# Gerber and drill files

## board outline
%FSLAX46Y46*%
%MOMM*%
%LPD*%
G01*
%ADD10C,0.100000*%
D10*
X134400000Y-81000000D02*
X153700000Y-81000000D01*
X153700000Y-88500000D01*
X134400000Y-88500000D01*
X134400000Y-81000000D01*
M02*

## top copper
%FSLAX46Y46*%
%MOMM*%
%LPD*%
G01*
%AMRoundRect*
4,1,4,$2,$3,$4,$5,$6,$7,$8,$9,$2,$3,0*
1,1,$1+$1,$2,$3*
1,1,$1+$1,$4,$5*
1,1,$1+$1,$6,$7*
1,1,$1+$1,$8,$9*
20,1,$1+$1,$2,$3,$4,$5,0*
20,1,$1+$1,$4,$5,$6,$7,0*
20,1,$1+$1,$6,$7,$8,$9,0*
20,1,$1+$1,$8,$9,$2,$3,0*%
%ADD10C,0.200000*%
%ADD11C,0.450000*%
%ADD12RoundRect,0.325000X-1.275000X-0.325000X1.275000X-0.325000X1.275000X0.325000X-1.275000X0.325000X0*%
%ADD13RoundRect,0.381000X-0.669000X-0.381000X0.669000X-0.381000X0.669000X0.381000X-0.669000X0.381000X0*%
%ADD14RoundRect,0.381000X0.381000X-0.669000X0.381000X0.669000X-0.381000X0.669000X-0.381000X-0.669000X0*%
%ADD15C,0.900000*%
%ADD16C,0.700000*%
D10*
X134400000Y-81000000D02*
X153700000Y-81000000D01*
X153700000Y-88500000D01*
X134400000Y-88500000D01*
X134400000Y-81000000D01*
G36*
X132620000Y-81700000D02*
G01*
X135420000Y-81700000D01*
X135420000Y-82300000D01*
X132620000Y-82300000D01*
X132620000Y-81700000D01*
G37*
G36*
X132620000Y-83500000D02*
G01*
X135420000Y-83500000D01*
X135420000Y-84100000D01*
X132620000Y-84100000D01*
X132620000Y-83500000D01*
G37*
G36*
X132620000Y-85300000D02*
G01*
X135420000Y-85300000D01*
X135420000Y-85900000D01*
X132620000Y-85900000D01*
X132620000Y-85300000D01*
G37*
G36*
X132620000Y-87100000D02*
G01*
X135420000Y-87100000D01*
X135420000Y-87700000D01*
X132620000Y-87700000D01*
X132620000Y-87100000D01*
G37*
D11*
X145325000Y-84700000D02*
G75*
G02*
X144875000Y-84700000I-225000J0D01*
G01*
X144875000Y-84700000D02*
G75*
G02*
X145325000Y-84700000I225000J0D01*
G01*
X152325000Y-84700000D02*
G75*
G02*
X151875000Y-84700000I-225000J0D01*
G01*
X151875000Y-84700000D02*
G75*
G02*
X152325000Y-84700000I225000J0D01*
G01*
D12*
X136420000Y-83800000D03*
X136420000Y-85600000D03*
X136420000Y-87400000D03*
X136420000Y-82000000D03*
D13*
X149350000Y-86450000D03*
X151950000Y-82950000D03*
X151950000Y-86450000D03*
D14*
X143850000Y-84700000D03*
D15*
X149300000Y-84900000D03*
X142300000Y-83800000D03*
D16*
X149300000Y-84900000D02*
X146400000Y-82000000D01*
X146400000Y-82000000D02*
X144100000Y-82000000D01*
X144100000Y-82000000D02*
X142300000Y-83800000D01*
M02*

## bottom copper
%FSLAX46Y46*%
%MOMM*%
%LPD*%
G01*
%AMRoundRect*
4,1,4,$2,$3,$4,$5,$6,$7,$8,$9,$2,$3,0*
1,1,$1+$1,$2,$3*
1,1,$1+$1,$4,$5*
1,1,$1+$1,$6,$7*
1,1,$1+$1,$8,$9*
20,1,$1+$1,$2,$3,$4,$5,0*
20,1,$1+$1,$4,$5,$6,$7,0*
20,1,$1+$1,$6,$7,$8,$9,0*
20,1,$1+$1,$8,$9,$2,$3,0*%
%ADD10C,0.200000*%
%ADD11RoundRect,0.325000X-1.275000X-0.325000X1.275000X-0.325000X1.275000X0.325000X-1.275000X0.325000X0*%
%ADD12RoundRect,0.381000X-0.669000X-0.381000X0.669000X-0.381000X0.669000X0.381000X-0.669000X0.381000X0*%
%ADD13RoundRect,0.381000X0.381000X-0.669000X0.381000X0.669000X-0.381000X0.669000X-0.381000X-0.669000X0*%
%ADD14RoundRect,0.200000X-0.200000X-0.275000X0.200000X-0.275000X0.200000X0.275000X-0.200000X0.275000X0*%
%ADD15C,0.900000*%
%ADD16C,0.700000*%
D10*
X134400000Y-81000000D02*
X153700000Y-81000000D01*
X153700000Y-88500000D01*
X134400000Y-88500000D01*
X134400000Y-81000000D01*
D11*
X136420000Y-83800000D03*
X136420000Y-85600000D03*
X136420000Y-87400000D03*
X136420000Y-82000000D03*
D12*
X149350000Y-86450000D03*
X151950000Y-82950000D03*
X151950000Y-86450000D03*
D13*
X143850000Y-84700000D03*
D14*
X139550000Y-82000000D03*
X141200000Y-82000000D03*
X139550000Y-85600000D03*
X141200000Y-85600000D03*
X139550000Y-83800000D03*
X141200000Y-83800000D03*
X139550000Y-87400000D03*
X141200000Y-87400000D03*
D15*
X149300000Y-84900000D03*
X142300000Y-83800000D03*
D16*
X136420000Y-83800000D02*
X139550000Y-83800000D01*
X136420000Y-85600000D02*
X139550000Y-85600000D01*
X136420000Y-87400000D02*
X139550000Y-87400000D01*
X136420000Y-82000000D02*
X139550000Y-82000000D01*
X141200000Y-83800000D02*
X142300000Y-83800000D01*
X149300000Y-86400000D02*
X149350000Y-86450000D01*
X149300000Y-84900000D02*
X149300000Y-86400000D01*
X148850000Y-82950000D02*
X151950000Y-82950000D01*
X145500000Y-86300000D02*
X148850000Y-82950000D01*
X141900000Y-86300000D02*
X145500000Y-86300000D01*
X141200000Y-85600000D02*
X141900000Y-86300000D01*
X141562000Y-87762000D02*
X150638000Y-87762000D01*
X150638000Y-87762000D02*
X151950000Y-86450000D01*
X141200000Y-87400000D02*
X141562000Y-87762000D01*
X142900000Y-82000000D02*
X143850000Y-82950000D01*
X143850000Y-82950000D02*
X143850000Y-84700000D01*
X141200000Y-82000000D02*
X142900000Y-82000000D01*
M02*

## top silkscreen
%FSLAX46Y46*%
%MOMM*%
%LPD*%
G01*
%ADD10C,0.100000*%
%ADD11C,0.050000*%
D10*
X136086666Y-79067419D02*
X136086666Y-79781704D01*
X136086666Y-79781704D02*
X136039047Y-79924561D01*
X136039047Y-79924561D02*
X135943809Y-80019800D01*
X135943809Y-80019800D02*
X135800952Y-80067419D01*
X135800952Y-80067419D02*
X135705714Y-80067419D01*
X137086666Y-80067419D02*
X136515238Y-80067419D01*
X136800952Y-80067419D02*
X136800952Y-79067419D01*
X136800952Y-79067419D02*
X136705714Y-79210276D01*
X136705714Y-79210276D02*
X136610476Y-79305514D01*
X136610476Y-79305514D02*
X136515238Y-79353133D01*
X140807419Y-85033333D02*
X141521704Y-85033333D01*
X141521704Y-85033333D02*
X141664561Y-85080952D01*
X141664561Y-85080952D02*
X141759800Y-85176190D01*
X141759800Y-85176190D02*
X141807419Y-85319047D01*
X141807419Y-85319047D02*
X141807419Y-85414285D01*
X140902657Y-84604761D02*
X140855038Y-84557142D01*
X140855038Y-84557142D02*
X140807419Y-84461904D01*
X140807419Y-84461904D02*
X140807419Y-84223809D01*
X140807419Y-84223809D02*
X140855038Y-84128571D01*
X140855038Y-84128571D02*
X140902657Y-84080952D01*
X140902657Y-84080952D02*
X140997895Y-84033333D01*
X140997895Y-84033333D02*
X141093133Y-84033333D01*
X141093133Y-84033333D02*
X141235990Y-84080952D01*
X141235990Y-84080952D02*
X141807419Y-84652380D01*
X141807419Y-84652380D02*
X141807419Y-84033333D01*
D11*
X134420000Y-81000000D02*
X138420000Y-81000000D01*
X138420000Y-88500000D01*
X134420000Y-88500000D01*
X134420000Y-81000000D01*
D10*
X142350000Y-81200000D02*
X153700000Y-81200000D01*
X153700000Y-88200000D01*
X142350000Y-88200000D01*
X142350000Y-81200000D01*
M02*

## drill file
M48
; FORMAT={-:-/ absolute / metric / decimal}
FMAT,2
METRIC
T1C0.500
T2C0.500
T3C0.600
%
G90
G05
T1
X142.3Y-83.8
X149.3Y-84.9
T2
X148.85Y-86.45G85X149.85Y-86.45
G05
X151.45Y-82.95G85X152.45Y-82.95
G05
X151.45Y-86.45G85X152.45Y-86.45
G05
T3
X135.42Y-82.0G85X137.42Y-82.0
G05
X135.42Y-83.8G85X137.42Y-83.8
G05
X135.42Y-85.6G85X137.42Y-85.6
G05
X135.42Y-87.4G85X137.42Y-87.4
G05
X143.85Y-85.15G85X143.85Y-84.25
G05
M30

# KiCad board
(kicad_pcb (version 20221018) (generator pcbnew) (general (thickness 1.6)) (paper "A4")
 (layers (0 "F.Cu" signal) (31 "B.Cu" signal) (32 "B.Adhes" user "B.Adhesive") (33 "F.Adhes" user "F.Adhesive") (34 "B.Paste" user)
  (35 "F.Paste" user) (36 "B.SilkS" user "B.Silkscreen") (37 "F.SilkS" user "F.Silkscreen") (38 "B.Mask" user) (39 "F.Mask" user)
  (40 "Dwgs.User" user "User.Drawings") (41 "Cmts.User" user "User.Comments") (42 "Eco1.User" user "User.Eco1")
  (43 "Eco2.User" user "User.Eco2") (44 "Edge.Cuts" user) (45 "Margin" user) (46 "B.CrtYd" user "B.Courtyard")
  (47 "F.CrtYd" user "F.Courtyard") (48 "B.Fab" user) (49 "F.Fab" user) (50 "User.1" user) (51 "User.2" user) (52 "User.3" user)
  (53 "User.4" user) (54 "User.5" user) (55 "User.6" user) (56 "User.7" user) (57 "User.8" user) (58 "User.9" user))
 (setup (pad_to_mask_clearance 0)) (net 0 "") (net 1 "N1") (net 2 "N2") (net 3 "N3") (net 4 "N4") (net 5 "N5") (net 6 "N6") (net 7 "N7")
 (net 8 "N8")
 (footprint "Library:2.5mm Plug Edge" (layer "F.Cu") (at 136.42 88.5)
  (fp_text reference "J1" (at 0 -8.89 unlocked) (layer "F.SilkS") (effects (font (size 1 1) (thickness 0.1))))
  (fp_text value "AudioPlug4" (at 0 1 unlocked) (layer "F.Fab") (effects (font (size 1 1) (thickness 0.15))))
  (fp_rect (start -3.8 -6.8) (end -1 -6.2) (stroke (width 0) (type solid)) (fill solid) (layer "F.Cu"))
  (fp_rect (start -3.8 -5) (end -1 -4.4) (stroke (width 0) (type solid)) (fill solid) (layer "F.Cu"))
  (fp_rect (start -3.8 -3.2) (end -1 -2.6) (stroke (width 0) (type solid)) (fill solid) (layer "F.Cu"))
  (fp_rect (start -3.8 -1.4) (end -1 -0.8) (stroke (width 0) (type solid)) (fill solid) (layer "F.Cu"))
  (fp_rect (start -2 -7.5) (end 2 0) (stroke (width 0.05) (type default)) (fill none) (layer "F.SilkS"))
  (pad "R1" thru_hole roundrect (at 0 -4.7) (size 3.2 1.3) (drill oval 2.6 0.6) (layers "*.Cu" "*.Mask") (roundrect_rratio 0.25)
   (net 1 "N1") (thermal_bridge_angle 45))
  (pad "R2" thru_hole roundrect (at 0 -2.9) (size 3.2 1.3) (drill oval 2.6 0.6) (layers "*.Cu" "*.Mask") (roundrect_rratio 0.25)
   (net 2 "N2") (thermal_bridge_angle 45))
  (pad "S" thru_hole roundrect (at 0 -1.1) (size 3.2 1.3) (drill oval 2.6 0.6) (layers "*.Cu" "*.Mask") (roundrect_rratio 0.25) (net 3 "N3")
   (thermal_bridge_angle 45))
  (pad "T" thru_hole roundrect (at 0 -6.5) (size 3.2 1.3) (drill oval 2.6 0.6) (layers "*.Cu" "*.Mask") (roundrect_rratio 0.25) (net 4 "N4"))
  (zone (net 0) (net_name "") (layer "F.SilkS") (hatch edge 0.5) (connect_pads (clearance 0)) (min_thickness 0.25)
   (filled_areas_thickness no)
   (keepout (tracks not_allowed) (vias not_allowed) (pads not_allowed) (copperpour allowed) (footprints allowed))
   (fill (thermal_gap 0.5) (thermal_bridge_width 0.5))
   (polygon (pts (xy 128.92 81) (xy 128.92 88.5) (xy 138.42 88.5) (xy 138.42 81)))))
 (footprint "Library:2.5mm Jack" (layer "F.Cu") (at 153.85 84.7 90)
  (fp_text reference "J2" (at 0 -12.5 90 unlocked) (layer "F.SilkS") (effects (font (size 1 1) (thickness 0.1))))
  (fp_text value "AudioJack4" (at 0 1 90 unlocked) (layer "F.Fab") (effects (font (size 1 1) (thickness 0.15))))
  (fp_circle (center 0 -8.75) (end 0.4 -8.75) (stroke (width 0.1) (type solid)) (fill solid) (layer "F.Cu"))
  (fp_circle (center 0 -1.75) (end 0.4 -1.75) (stroke (width 0.1) (type solid)) (fill solid) (layer "F.Cu"))
  (fp_rect (start -3.5 -11.5) (end 3.5 -0.15) (stroke (width 0.1) (type default)) (fill none) (layer "F.SilkS"))
  (pad "R1" thru_hole roundrect (at -1.75 -4.5) (size 2.1 1.524) (drill oval 1.5 0.5) (layers "*.Cu" "*.Mask") (roundrect_rratio 0.25)
   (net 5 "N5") (thermal_bridge_angle 45))
  (pad "R2" thru_hole roundrect (at 1.75 -1.9) (size 2.1 1.524) (drill oval 1.5 0.5) (layers "*.Cu" "*.Mask") (roundrect_rratio 0.25)
   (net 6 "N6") (thermal_bridge_angle 45))
  (pad "S" thru_hole roundrect (at -1.75 -1.9) (size 2.1 1.524) (drill oval 1.5 0.5) (layers "*.Cu" "*.Mask") (roundrect_rratio 0.25)
   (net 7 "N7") (thermal_bridge_angle 45))
  (pad "T" thru_hole roundrect (at 0 -10 90) (size 2.1 1.524) (drill oval 1.5 0.6) (layers "*.Cu" "*.Mask") (roundrect_rratio 0.25)
   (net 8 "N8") (thermal_bridge_angle 45))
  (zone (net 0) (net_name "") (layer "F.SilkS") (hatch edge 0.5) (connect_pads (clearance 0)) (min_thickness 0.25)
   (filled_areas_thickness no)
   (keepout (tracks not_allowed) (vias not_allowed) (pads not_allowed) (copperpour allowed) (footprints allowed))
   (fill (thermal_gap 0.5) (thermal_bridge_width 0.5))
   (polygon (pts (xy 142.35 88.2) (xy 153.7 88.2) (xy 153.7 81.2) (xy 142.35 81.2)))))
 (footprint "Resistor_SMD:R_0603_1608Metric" (layer "B.Cu") (at 140.375 82)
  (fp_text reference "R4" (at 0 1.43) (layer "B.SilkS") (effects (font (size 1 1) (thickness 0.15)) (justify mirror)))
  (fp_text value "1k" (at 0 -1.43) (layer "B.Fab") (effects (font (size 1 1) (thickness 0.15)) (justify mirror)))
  (pad "1" smd roundrect (at -0.825 0) (size 0.8 0.95) (layers "B.Cu" "B.Paste" "B.Mask") (roundrect_rratio 0.25) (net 4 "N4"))
  (pad "2" smd roundrect (at 0.825 0) (size 0.8 0.95) (layers "B.Cu" "B.Paste" "B.Mask") (roundrect_rratio 0.25) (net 8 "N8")))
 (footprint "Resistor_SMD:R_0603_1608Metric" (layer "B.Cu") (at 140.375 85.6)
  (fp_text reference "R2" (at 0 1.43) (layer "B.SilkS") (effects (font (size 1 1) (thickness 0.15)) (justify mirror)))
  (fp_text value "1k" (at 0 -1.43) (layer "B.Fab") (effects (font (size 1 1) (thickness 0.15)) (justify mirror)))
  (pad "1" smd roundrect (at -0.825 0) (size 0.8 0.95) (layers "B.Cu" "B.Paste" "B.Mask") (roundrect_rratio 0.25) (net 2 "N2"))
  (pad "2" smd roundrect (at 0.825 0) (size 0.8 0.95) (layers "B.Cu" "B.Paste" "B.Mask") (roundrect_rratio 0.25) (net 6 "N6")))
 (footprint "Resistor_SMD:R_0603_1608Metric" (layer "B.Cu") (at 140.375 83.8)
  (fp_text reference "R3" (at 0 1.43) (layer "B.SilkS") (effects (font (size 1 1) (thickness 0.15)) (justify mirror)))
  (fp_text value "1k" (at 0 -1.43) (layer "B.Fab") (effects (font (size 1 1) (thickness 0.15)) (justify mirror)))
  (pad "1" smd roundrect (at -0.825 0) (size 0.8 0.95) (layers "B.Cu" "B.Paste" "B.Mask") (roundrect_rratio 0.25) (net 1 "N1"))
  (pad "2" smd roundrect (at 0.825 0) (size 0.8 0.95) (layers "B.Cu" "B.Paste" "B.Mask") (roundrect_rratio 0.25) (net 5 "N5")))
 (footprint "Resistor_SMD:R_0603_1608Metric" (layer "B.Cu") (at 140.375 87.4)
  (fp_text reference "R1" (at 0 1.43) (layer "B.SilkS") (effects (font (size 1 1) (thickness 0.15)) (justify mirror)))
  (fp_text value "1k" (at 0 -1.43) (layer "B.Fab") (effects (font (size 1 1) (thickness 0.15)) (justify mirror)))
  (pad "1" smd roundrect (at -0.825 0) (size 0.8 0.95) (layers "B.Cu" "B.Paste" "B.Mask") (roundrect_rratio 0.25) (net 3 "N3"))
  (pad "2" smd roundrect (at 0.825 0) (size 0.8 0.95) (layers "B.Cu" "B.Paste" "B.Mask") (roundrect_rratio 0.25) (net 7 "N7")))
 (gr_rect (start 134.4 81) (end 153.7 88.5) (stroke (width 0.2) (type default)) (fill none) (layer "F.Cu"))
 (gr_rect (start 134.4 81) (end 153.7 88.5) (stroke (width 0.2) (type default)) (fill none) (layer "B.Cu"))
 (gr_rect (start 134.4 81) (end 153.7 88.5) (stroke (width 0.1) (type default)) (fill none) (layer "Edge.Cuts"))
 (segment (start 136.42 83.8) (end 139.55 83.8) (width 0.7) (layer "B.Cu") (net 1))
 (segment (start 136.42 85.6) (end 139.55 85.6) (width 0.7) (layer "B.Cu") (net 2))
 (segment (start 136.42 87.4) (end 139.55 87.4) (width 0.7) (layer "B.Cu") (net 3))
 (segment (start 136.42 82) (end 139.55 82) (width 0.7) (layer "B.Cu") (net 4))
 (segment (start 149.3 84.9) (end 146.4 82) (width 0.7) (layer "F.Cu") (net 5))
 (segment (start 146.4 82) (end 144.1 82) (width 0.7) (layer "F.Cu") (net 5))
 (segment (start 144.1 82) (end 142.3 83.8) (width 0.7) (layer "F.Cu") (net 5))
 (via (at 149.3 84.9) (size 0.9) (drill 0.5) (layers "F.Cu" "B.Cu") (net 5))
 (via (at 142.3 83.8) (size 0.9) (drill 0.5) (layers "F.Cu" "B.Cu") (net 5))
 (segment (start 141.2 83.8) (end 142.3 83.8) (width 0.7) (layer "B.Cu") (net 5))
 (segment (start 149.3 86.4) (end 149.35 86.45) (width 0.7) (layer "B.Cu") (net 5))
 (segment (start 149.3 84.9) (end 149.3 86.4) (width 0.7) (layer "B.Cu") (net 5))
 (segment (start 148.85 82.95) (end 151.95 82.95) (width 0.7) (layer "B.Cu") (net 6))
 (segment (start 145.5 86.3) (end 148.85 82.95) (width 0.7) (layer "B.Cu") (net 6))
 (segment (start 141.9 86.3) (end 145.5 86.3) (width 0.7) (layer "B.Cu") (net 6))
 (segment (start 141.2 85.6) (end 141.9 86.3) (width 0.7) (layer "B.Cu") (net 6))
 (segment (start 141.562 87.762) (end 150.638 87.762) (width 0.7) (layer "B.Cu") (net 7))
 (segment (start 150.638 87.762) (end 151.95 86.45) (width 0.7) (layer "B.Cu") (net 7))
 (segment (start 141.2 87.4) (end 141.562 87.762) (width 0.7) (layer "B.Cu") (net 7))
 (segment (start 142.9 82) (end 143.85 82.95) (width 0.7) (layer "B.Cu") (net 8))
 (segment (start 143.85 82.95) (end 143.85 84.7) (width 0.7) (layer "B.Cu") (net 8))
 (segment (start 141.2 82) (end 142.9 82) (width 0.7) (layer "B.Cu") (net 8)))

